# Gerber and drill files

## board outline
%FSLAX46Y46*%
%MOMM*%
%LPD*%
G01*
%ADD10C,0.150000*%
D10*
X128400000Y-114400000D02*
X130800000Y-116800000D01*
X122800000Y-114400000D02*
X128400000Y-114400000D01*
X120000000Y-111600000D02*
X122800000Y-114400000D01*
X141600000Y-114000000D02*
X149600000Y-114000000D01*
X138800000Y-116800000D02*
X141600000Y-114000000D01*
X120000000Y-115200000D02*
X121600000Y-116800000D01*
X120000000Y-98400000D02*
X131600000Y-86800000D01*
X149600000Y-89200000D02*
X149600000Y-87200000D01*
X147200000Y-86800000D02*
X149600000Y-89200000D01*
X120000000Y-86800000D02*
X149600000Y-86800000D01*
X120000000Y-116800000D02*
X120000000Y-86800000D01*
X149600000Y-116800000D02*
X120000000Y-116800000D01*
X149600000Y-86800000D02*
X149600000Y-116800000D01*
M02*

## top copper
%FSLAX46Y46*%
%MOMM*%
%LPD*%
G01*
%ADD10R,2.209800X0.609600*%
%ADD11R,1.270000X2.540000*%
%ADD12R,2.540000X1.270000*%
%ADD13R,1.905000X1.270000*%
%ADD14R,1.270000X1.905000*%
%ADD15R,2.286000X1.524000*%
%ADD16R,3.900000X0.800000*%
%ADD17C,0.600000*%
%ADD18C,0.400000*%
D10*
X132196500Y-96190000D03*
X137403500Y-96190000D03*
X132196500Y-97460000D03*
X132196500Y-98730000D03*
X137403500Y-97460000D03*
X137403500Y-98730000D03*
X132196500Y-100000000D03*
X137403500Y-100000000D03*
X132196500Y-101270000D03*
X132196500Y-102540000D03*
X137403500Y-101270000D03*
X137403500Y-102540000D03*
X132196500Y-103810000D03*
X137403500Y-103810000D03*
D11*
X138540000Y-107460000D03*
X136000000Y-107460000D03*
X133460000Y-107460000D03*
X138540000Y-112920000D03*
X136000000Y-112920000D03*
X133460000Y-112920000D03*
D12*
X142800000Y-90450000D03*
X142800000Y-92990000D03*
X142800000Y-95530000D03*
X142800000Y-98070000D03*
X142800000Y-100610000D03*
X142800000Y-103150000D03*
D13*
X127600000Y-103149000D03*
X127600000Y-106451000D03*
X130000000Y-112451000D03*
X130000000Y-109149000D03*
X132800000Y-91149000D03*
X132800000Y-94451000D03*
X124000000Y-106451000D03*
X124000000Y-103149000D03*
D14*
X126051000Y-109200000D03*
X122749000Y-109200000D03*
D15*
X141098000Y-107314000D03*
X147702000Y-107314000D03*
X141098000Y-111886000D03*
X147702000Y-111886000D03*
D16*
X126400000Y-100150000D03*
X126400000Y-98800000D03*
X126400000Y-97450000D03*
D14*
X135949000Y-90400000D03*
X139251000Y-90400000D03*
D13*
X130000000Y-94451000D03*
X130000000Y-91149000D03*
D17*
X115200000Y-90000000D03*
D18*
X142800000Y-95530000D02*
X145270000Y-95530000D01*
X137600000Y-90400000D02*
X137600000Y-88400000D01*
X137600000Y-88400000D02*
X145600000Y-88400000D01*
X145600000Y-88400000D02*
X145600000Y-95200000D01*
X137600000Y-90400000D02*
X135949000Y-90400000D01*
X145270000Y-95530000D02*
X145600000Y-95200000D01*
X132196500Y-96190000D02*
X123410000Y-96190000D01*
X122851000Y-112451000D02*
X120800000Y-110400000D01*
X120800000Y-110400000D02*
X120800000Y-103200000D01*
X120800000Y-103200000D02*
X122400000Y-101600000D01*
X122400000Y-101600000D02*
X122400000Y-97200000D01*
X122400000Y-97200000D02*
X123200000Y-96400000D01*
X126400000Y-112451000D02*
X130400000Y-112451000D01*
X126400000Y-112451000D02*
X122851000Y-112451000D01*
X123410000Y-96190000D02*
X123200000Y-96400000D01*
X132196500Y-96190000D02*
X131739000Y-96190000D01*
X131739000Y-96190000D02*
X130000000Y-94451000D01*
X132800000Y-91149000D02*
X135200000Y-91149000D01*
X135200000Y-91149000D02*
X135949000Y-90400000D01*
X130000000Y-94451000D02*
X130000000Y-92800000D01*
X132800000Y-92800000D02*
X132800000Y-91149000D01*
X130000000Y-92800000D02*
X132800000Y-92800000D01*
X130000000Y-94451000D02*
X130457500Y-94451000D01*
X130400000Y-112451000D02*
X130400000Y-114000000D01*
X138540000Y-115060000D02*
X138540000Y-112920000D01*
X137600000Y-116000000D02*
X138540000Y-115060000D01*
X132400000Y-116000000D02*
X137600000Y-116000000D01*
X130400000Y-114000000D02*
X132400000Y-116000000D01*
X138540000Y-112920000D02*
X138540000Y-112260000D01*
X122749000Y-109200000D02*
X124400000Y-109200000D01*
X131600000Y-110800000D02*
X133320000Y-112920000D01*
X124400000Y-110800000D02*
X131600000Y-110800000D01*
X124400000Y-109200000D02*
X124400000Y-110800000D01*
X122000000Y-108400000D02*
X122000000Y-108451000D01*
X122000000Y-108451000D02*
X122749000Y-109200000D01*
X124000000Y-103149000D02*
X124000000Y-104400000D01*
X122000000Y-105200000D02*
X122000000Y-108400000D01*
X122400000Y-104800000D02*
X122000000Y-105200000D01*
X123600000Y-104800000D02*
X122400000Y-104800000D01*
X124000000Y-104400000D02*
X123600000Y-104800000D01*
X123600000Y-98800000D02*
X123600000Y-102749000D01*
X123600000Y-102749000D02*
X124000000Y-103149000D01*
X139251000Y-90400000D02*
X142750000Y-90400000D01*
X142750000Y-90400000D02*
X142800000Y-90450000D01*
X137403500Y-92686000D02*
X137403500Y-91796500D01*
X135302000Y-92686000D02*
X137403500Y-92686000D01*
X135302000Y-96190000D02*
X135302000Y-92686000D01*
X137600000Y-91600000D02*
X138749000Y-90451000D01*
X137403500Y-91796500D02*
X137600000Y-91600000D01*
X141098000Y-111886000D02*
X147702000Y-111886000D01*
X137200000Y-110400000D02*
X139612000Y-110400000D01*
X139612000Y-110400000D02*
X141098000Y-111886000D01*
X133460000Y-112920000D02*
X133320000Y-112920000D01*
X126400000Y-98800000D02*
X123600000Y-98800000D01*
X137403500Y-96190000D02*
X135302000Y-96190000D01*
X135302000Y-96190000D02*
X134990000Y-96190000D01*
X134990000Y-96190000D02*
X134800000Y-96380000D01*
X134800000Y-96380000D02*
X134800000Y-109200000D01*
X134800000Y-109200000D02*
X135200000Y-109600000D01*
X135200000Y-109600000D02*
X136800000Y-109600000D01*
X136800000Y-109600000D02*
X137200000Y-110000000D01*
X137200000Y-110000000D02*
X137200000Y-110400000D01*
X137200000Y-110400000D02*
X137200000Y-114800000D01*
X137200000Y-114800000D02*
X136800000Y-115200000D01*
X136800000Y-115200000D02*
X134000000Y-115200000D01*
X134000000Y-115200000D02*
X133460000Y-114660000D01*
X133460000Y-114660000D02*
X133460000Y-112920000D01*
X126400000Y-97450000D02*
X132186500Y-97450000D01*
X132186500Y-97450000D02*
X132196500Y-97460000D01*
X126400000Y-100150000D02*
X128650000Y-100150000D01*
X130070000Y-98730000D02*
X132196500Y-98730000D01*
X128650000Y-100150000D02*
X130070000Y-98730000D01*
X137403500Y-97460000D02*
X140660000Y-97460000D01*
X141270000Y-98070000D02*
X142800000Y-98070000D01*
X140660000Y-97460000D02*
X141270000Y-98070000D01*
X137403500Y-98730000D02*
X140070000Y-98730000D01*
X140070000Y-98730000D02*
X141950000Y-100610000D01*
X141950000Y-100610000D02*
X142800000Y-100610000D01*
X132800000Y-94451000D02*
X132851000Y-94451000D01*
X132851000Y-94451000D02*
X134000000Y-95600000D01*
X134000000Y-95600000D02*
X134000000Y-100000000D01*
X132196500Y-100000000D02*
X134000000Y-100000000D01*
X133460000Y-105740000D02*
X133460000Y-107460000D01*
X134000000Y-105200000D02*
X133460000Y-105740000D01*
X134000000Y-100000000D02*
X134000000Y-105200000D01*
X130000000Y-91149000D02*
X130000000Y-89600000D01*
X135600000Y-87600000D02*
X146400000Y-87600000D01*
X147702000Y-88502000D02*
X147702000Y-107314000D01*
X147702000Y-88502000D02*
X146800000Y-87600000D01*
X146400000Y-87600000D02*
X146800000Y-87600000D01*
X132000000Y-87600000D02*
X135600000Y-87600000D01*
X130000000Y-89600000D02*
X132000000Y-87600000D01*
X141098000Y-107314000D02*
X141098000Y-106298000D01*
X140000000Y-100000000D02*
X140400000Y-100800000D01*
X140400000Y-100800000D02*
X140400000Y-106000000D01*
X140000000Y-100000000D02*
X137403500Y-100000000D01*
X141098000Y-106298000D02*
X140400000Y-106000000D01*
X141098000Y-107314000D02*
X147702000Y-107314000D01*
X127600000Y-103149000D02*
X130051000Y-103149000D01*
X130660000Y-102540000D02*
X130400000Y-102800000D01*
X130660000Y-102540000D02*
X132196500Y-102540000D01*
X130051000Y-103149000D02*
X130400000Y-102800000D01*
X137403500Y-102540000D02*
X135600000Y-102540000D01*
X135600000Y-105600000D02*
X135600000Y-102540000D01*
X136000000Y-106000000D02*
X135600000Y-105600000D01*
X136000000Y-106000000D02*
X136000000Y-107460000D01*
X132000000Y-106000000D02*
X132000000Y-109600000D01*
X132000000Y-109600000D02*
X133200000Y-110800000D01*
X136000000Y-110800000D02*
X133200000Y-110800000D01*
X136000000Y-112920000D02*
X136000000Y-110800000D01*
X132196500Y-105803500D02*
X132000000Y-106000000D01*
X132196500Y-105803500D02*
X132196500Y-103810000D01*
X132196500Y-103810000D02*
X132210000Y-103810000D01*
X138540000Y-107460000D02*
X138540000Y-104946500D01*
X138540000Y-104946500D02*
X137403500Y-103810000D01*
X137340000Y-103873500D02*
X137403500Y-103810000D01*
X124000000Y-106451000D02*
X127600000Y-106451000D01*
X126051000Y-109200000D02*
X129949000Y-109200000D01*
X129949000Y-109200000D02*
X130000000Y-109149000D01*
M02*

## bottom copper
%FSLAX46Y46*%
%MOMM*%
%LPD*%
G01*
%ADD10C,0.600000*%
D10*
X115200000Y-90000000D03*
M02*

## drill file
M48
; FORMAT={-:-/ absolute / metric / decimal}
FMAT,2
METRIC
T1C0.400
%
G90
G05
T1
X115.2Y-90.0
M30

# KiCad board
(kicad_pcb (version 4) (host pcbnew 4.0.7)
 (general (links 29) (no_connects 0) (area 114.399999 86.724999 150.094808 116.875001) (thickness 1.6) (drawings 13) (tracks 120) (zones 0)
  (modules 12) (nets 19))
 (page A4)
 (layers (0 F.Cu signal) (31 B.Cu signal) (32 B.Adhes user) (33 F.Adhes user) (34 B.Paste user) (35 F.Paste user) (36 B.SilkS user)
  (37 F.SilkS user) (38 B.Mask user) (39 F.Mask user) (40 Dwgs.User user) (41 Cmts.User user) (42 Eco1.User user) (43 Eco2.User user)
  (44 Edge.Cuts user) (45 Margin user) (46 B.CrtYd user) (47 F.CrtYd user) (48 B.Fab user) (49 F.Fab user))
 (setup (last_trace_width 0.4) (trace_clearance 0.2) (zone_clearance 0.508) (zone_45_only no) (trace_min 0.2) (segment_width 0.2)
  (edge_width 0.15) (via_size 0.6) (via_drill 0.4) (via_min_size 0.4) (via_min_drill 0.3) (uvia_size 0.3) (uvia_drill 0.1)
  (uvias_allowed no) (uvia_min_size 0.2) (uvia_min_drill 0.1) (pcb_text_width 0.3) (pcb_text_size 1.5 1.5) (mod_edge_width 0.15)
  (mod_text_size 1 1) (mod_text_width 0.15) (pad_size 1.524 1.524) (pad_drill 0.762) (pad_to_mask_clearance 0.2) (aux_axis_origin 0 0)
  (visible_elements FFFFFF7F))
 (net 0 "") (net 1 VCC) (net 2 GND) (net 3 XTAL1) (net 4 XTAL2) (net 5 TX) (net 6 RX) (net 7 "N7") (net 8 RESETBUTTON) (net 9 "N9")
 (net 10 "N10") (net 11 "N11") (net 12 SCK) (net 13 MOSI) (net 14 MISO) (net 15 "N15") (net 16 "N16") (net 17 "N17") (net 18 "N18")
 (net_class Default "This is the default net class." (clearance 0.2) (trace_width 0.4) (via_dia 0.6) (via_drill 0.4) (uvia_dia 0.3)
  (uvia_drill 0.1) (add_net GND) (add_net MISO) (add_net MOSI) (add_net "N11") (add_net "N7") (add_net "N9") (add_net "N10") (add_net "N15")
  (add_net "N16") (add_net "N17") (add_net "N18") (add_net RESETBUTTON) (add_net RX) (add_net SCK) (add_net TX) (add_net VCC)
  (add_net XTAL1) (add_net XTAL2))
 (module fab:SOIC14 (layer F.Cu) (at 134.8 100 270)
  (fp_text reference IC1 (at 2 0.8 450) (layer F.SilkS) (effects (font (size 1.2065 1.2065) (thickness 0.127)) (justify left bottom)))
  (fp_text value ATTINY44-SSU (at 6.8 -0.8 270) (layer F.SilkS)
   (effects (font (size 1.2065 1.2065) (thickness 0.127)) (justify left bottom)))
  (pad 1 smd rect (at -3.81 2.6035 270) (size 0.6096 2.2098) (layers F.Cu F.Paste F.Mask) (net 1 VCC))
  (pad 14 smd rect (at -3.81 -2.6035 270) (size 0.6096 2.2098) (layers F.Cu F.Paste F.Mask) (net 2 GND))
  (pad 2 smd rect (at -2.54 2.6035 270) (size 0.6096 2.2098) (layers F.Cu F.Paste F.Mask) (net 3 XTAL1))
  (pad 3 smd rect (at -1.27 2.6035 270) (size 0.6096 2.2098) (layers F.Cu F.Paste F.Mask) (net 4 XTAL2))
  (pad 13 smd rect (at -2.54 -2.6035 270) (size 0.6096 2.2098) (layers F.Cu F.Paste F.Mask) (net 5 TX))
  (pad 12 smd rect (at -1.27 -2.6035 270) (size 0.6096 2.2098) (layers F.Cu F.Paste F.Mask) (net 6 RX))
  (pad 4 smd rect (at 0 2.6035 270) (size 0.6096 2.2098) (layers F.Cu F.Paste F.Mask) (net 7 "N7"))
  (pad 11 smd rect (at 0 -2.6035 270) (size 0.6096 2.2098) (layers F.Cu F.Paste F.Mask) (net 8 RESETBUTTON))
  (pad 5 smd rect (at 1.27 2.6035 270) (size 0.6096 2.2098) (layers F.Cu F.Paste F.Mask) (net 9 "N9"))
  (pad 6 smd rect (at 2.54 2.6035 270) (size 0.6096 2.2098) (layers F.Cu F.Paste F.Mask) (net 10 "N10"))
  (pad 10 smd rect (at 1.27 -2.6035 270) (size 0.6096 2.2098) (layers F.Cu F.Paste F.Mask) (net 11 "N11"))
  (pad 9 smd rect (at 2.54 -2.6035 270) (size 0.6096 2.2098) (layers F.Cu F.Paste F.Mask) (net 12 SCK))
  (pad 7 smd rect (at 3.81 2.6035 270) (size 0.6096 2.2098) (layers F.Cu F.Paste F.Mask) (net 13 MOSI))
  (pad 8 smd rect (at 3.81 -2.6035 270) (size 0.6096 2.2098) (layers F.Cu F.Paste F.Mask) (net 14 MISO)))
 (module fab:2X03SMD (layer F.Cu) (at 136 110 270)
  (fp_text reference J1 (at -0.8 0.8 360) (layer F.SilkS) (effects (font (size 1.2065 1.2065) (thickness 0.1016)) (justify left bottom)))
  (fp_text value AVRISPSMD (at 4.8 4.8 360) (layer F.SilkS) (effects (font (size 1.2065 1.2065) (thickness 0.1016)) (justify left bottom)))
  (pad 1 smd rect (at -2.54 -2.54 270) (size 2.54 1.27) (layers F.Cu F.Paste F.Mask) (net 14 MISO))
  (pad 3 smd rect (at -2.54 0 270) (size 2.54 1.27) (layers F.Cu F.Paste F.Mask) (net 12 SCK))
  (pad 5 smd rect (at -2.54 2.54 270) (size 2.54 1.27) (layers F.Cu F.Paste F.Mask) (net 7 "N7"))
  (pad 2 smd rect (at 2.92 -2.54 270) (size 2.54 1.27) (layers F.Cu F.Paste F.Mask) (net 1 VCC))
  (pad 4 smd rect (at 2.92 0 270) (size 2.54 1.27) (layers F.Cu F.Paste F.Mask) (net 13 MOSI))
  (pad 6 smd rect (at 2.92 2.54 270) (size 2.54 1.27) (layers F.Cu F.Paste F.Mask) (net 2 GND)))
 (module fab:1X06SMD (layer F.Cu) (at 142.8 96.8)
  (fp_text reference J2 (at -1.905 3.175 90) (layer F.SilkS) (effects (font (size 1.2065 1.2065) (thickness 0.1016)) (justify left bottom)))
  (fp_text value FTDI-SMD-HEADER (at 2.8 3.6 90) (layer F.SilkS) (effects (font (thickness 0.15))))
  (pad 1 smd rect (at 0 -6.35) (size 2.54 1.27) (layers F.Cu F.Paste F.Mask) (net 2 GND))
  (pad 2 smd rect (at 0 -3.81) (size 2.54 1.27) (layers F.Cu F.Paste F.Mask) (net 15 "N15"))
  (pad 3 smd rect (at 0 -1.27) (size 2.54 1.27) (layers F.Cu F.Paste F.Mask) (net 1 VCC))
  (pad 4 smd rect (at 0 1.27) (size 2.54 1.27) (layers F.Cu F.Paste F.Mask) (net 5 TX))
  (pad 5 smd rect (at 0 3.81) (size 2.54 1.27) (layers F.Cu F.Paste F.Mask) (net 6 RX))
  (pad 6 smd rect (at 0 6.35) (size 2.54 1.27) (layers F.Cu F.Paste F.Mask) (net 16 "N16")))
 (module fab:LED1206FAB (layer F.Cu) (at 127.6 104.8 270)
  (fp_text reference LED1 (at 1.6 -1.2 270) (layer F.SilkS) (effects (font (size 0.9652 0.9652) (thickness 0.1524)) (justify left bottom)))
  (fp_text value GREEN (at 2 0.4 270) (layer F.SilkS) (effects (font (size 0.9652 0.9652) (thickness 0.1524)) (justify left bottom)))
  (pad 1 smd rect (at -1.651 0 270) (size 1.27 1.905) (layers F.Cu F.Paste F.Mask) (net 10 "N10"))
  (pad 2 smd rect (at 1.651 0 270) (size 1.27 1.905) (layers F.Cu F.Paste F.Mask) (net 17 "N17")))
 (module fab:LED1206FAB (layer F.Cu) (at 130 110.8 90)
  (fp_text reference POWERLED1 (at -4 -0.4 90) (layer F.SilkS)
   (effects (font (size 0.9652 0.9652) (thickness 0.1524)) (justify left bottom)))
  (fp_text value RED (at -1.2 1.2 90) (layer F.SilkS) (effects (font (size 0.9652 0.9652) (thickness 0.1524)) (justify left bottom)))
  (pad 1 smd rect (at -1.651 0 90) (size 1.27 1.905) (layers F.Cu F.Paste F.Mask) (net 1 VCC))
  (pad 2 smd rect (at 1.651 0 90) (size 1.27 1.905) (layers F.Cu F.Paste F.Mask) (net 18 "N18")))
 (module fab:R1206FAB (layer F.Cu) (at 132.8 92.8 270)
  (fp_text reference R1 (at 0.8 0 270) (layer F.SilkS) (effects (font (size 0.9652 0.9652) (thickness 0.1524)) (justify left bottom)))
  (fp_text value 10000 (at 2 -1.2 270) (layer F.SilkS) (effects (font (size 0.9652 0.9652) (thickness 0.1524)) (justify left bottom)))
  (pad 1 smd rect (at -1.651 0 270) (size 1.27 1.905) (layers F.Cu F.Paste F.Mask) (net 1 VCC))
  (pad 2 smd rect (at 1.651 0 270) (size 1.27 1.905) (layers F.Cu F.Paste F.Mask) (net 7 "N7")))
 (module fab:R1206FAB (layer F.Cu) (at 124 104.8 90)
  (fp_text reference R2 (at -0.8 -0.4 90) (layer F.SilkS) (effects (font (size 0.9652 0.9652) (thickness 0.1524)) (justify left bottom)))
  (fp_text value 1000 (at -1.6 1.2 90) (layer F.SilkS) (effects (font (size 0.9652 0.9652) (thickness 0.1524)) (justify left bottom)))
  (pad 1 smd rect (at -1.651 0 90) (size 1.27 1.905) (layers F.Cu F.Paste F.Mask) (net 17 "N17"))
  (pad 2 smd rect (at 1.651 0 90) (size 1.27 1.905) (layers F.Cu F.Paste F.Mask) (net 2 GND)))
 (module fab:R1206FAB (layer F.Cu) (at 124.4 109.2 180)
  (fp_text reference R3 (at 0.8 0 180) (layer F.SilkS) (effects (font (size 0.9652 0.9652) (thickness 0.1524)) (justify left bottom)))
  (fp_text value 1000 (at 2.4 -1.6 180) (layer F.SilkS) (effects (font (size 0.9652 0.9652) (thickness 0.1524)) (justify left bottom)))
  (pad 1 smd rect (at -1.651 0 180) (size 1.27 1.905) (layers F.Cu F.Paste F.Mask) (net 18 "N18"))
  (pad 2 smd rect (at 1.651 0 180) (size 1.27 1.905) (layers F.Cu F.Paste F.Mask) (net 2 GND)))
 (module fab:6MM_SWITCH (layer F.Cu) (at 144.4 109.6)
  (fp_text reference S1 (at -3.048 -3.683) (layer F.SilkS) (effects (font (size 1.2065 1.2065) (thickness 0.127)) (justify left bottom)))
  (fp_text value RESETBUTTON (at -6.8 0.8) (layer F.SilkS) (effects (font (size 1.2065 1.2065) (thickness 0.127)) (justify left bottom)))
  (pad 1 smd rect (at -3.302 -2.286) (size 2.286 1.524) (layers F.Cu F.Paste F.Mask) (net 8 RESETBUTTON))
  (pad 2 smd rect (at 3.302 -2.286) (size 2.286 1.524) (layers F.Cu F.Paste F.Mask) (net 8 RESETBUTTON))
  (pad 3 smd rect (at -3.302 2.286) (size 2.286 1.524) (layers F.Cu F.Paste F.Mask) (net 2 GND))
  (pad 4 smd rect (at 3.302 2.286) (size 2.286 1.524) (layers F.Cu F.Paste F.Mask) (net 2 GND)))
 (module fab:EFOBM (layer F.Cu) (at 126.4 98.8 90)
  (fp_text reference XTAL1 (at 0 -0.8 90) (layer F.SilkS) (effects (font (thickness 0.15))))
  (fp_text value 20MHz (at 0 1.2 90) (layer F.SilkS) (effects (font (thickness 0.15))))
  (pad 1 smd rect (at -1.35 0 180) (size 3.9 0.8) (layers F.Cu F.Paste F.Mask) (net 4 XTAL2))
  (pad 2 smd rect (at 0 0) (size 3.9 0.8) (layers F.Cu F.Paste F.Mask) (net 2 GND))
  (pad 3 smd rect (at 1.35 0) (size 3.9 0.8) (layers F.Cu F.Paste F.Mask) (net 3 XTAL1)))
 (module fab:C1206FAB (layer F.Cu) (at 137.6 90.4)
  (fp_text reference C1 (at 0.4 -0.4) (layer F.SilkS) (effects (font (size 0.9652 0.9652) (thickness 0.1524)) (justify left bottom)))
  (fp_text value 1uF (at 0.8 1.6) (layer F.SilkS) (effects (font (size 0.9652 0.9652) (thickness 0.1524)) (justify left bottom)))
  (pad 1 smd rect (at -1.651 0) (size 1.27 1.905) (layers F.Cu F.Paste F.Mask) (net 1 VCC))
  (pad 2 smd rect (at 1.651 0) (size 1.27 1.905) (layers F.Cu F.Paste F.Mask) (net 2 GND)))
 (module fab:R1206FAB (layer F.Cu) (at 130 92.8 90)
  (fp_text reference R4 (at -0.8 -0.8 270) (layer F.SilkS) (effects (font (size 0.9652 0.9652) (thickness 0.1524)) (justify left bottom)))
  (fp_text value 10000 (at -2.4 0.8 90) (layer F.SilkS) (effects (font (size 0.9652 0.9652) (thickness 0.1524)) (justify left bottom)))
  (pad 1 smd rect (at -1.651 0 90) (size 1.27 1.905) (layers F.Cu F.Paste F.Mask) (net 1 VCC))
  (pad 2 smd rect (at 1.651 0 90) (size 1.27 1.905) (layers F.Cu F.Paste F.Mask) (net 8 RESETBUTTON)))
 (gr_line (start 128.4 114.4) (end 130.8 116.8) (angle 90) (layer Edge.Cuts) (width 0.15))
 (gr_line (start 122.8 114.4) (end 128.4 114.4) (angle 90) (layer Edge.Cuts) (width 0.15))
 (gr_line (start 120 111.6) (end 122.8 114.4) (angle 90) (layer Edge.Cuts) (width 0.15))
 (gr_line (start 141.6 114) (end 149.6 114) (angle 90) (layer Edge.Cuts) (width 0.15))
 (gr_line (start 138.8 116.8) (end 141.6 114) (angle 90) (layer Edge.Cuts) (width 0.15))
 (gr_line (start 120 115.2) (end 121.6 116.8) (angle 90) (layer Edge.Cuts) (width 0.15))
 (gr_line (start 120 98.4) (end 131.6 86.8) (angle 90) (layer Edge.Cuts) (width 0.15))
 (gr_line (start 149.6 89.2) (end 149.6 87.2) (angle 90) (layer Edge.Cuts) (width 0.15))
 (gr_line (start 147.2 86.8) (end 149.6 89.2) (angle 90) (layer Edge.Cuts) (width 0.15))
 (gr_line (start 120 86.8) (end 149.6 86.8) (angle 90) (layer Edge.Cuts) (width 0.15))
 (gr_line (start 120 116.8) (end 120 86.8) (angle 90) (layer Edge.Cuts) (width 0.15))
 (gr_line (start 149.6 116.8) (end 120 116.8) (angle 90) (layer Edge.Cuts) (width 0.15))
 (gr_line (start 149.6 86.8) (end 149.6 116.8) (angle 90) (layer Edge.Cuts) (width 0.15))
 (via (at 115.2 90) (size 0.6) (drill 0.4) (layers F.Cu B.Cu) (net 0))
 (segment (start 142.8 95.53) (end 145.27 95.53) (width 0.4) (layer F.Cu) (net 1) (status 400000))
 (segment (start 137.6 90.4) (end 137.6 88.4) (width 0.4) (layer F.Cu) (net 1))
 (segment (start 137.6 88.4) (end 145.6 88.4) (width 0.4) (layer F.Cu) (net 1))
 (segment (start 145.6 88.4) (end 145.6 95.2) (width 0.4) (layer F.Cu) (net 1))
 (segment (start 137.6 90.4) (end 135.949 90.4) (width 0.4) (layer F.Cu) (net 1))
 (segment (start 145.27 95.53) (end 145.6 95.2) (width 0.4) (layer F.Cu) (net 1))
 (segment (start 132.1965 96.19) (end 123.41 96.19) (width 0.4) (layer F.Cu) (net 1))
 (segment (start 122.851 112.451) (end 120.8 110.4) (width 0.4) (layer F.Cu) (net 1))
 (segment (start 120.8 110.4) (end 120.8 103.2) (width 0.4) (layer F.Cu) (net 1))
 (segment (start 120.8 103.2) (end 122.4 101.6) (width 0.4) (layer F.Cu) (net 1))
 (segment (start 122.4 101.6) (end 122.4 97.2) (width 0.4) (layer F.Cu) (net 1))
 (segment (start 122.4 97.2) (end 123.2 96.4) (width 0.4) (layer F.Cu) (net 1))
 (segment (start 126.4 112.451) (end 130.4 112.451) (width 0.4) (layer F.Cu) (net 1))
 (segment (start 126.4 112.451) (end 122.851 112.451) (width 0.4) (layer F.Cu) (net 1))
 (segment (start 123.41 96.19) (end 123.2 96.4) (width 0.4) (layer F.Cu) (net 1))
 (segment (start 132.1965 96.19) (end 131.739 96.19) (width 0.4) (layer F.Cu) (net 1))
 (segment (start 131.739 96.19) (end 130 94.451) (width 0.4) (layer F.Cu) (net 1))
 (segment (start 132.8 91.149) (end 135.2 91.149) (width 0.4) (layer F.Cu) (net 1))
 (segment (start 135.2 91.149) (end 135.949 90.4) (width 0.4) (layer F.Cu) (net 1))
 (segment (start 130 94.451) (end 130 92.8) (width 0.4) (layer F.Cu) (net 1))
 (segment (start 132.8 92.8) (end 132.8 91.149) (width 0.4) (layer F.Cu) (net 1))
 (segment (start 130 92.8) (end 132.8 92.8) (width 0.4) (layer F.Cu) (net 1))
 (segment (start 130 94.451) (end 130.4575 94.451) (width 0.4) (layer F.Cu) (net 1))
 (segment (start 130.4 112.451) (end 130.4 114) (width 0.4) (layer F.Cu) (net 1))
 (segment (start 138.54 115.06) (end 138.54 112.92) (width 0.4) (layer F.Cu) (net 1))
 (segment (start 137.6 116) (end 138.54 115.06) (width 0.4) (layer F.Cu) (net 1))
 (segment (start 132.4 116) (end 137.6 116) (width 0.4) (layer F.Cu) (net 1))
 (segment (start 130.4 114) (end 132.4 116) (width 0.4) (layer F.Cu) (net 1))
 (segment (start 138.54 112.92) (end 138.54 112.26) (width 0.4) (layer F.Cu) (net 1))
 (segment (start 122.749 109.2) (end 124.4 109.2) (width 0.4) (layer F.Cu) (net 2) (status 400000))
 (segment (start 131.6 110.8) (end 133.32 112.92) (width 0.4) (layer F.Cu) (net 2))
 (segment (start 124.4 110.8) (end 131.6 110.8) (width 0.4) (layer F.Cu) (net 2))
 (segment (start 124.4 109.2) (end 124.4 110.8) (width 0.4) (layer F.Cu) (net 2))
 (segment (start 122 108.4) (end 122 108.451) (width 0.4) (layer F.Cu) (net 2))
 (segment (start 122 108.451) (end 122.749 109.2) (width 0.4) (layer F.Cu) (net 2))
 (segment (start 124 103.149) (end 124 104.4) (width 0.4) (layer F.Cu) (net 2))
 (segment (start 122 105.2) (end 122 108.4) (width 0.4) (layer F.Cu) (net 2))
 (segment (start 122.4 104.8) (end 122 105.2) (width 0.4) (layer F.Cu) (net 2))
 (segment (start 123.6 104.8) (end 122.4 104.8) (width 0.4) (layer F.Cu) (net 2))
 (segment (start 124 104.4) (end 123.6 104.8) (width 0.4) (layer F.Cu) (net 2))
 (segment (start 123.6 98.8) (end 123.6 102.749) (width 0.4) (layer F.Cu) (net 2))
 (segment (start 123.6 102.749) (end 124 103.149) (width 0.4) (layer F.Cu) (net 2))
 (segment (start 139.251 90.4) (end 142.75 90.4) (width 0.4) (layer F.Cu) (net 2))
 (segment (start 142.75 90.4) (end 142.8 90.45) (width 0.4) (layer F.Cu) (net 2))
 (segment (start 137.4035 92.686) (end 137.4035 91.7965) (width 0.4) (layer F.Cu) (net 2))
 (segment (start 135.302 92.686) (end 137.4035 92.686) (width 0.4) (layer F.Cu) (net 2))
 (segment (start 135.302 96.19) (end 135.302 92.686) (width 0.4) (layer F.Cu) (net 2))
 (segment (start 137.6 91.6) (end 138.749 90.451) (width 0.4) (layer F.Cu) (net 2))
 (segment (start 137.4035 91.7965) (end 137.6 91.6) (width 0.4) (layer F.Cu) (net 2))
 (segment (start 141.098 111.886) (end 147.702 111.886) (width 0.4) (layer F.Cu) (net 2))
 (segment (start 137.2 110.4) (end 139.612 110.4) (width 0.4) (layer F.Cu) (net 2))
 (segment (start 139.612 110.4) (end 141.098 111.886) (width 0.4) (layer F.Cu) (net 2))
 (segment (start 133.46 112.92) (end 133.32 112.92) (width 0.4) (layer F.Cu) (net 2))
 (segment (start 126.4 98.8) (end 123.6 98.8) (width 0.4) (layer F.Cu) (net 2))
 (segment (start 137.4035 96.19) (end 135.302 96.19) (width 0.4) (layer F.Cu) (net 2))
 (segment (start 135.302 96.19) (end 134.99 96.19) (width 0.4) (layer F.Cu) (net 2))
 (segment (start 134.99 96.19) (end 134.8 96.38) (width 0.4) (layer F.Cu) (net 2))
 (segment (start 134.8 96.38) (end 134.8 109.2) (width 0.4) (layer F.Cu) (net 2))
 (segment (start 134.8 109.2) (end 135.2 109.6) (width 0.4) (layer F.Cu) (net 2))
 (segment (start 135.2 109.6) (end 136.8 109.6) (width 0.4) (layer F.Cu) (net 2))
 (segment (start 136.8 109.6) (end 137.2 110) (width 0.4) (layer F.Cu) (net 2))
 (segment (start 137.2 110) (end 137.2 110.4) (width 0.4) (layer F.Cu) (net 2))
 (segment (start 137.2 110.4) (end 137.2 114.8) (width 0.4) (layer F.Cu) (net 2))
 (segment (start 137.2 114.8) (end 136.8 115.2) (width 0.4) (layer F.Cu) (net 2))
 (segment (start 136.8 115.2) (end 134 115.2) (width 0.4) (layer F.Cu) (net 2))
 (segment (start 134 115.2) (end 133.46 114.66) (width 0.4) (layer F.Cu) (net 2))
 (segment (start 133.46 114.66) (end 133.46 112.92) (width 0.4) (layer F.Cu) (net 2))
 (segment (start 126.4 97.45) (end 132.1865 97.45) (width 0.4) (layer F.Cu) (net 3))
 (segment (start 132.1865 97.45) (end 132.1965 97.46) (width 0.4) (layer F.Cu) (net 3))
 (segment (start 126.4 100.15) (end 128.65 100.15) (width 0.4) (layer F.Cu) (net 4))
 (segment (start 130.07 98.73) (end 132.1965 98.73) (width 0.4) (layer F.Cu) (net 4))
 (segment (start 128.65 100.15) (end 130.07 98.73) (width 0.4) (layer F.Cu) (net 4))
 (segment (start 137.4035 97.46) (end 140.66 97.46) (width 0.4) (layer F.Cu) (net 5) (status 400000))
 (segment (start 141.27 98.07) (end 142.8 98.07) (width 0.4) (layer F.Cu) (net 5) (status 800000))
 (segment (start 140.66 97.46) (end 141.27 98.07) (width 0.4) (layer F.Cu) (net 5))
 (segment (start 137.4035 98.73) (end 140.07 98.73) (width 0.4) (layer F.Cu) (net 6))
 (segment (start 140.07 98.73) (end 141.95 100.61) (width 0.4) (layer F.Cu) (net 6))
 (segment (start 141.95 100.61) (end 142.8 100.61) (width 0.4) (layer F.Cu) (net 6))
 (segment (start 132.8 94.451) (end 132.851 94.451) (width 0.4) (layer F.Cu) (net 7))
 (segment (start 132.851 94.451) (end 134 95.6) (width 0.4) (layer F.Cu) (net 7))
 (segment (start 134 95.6) (end 134 100) (width 0.4) (layer F.Cu) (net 7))
 (segment (start 132.1965 100) (end 134 100) (width 0.4) (layer F.Cu) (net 7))
 (segment (start 133.46 105.74) (end 133.46 107.46) (width 0.4) (layer F.Cu) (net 7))
 (segment (start 134 105.2) (end 133.46 105.74) (width 0.4) (layer F.Cu) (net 7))
 (segment (start 134 100) (end 134 105.2) (width 0.4) (layer F.Cu) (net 7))
 (segment (start 130 91.149) (end 130 89.6) (width 0.4) (layer F.Cu) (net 8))
 (segment (start 135.6 87.6) (end 146.4 87.6) (width 0.4) (layer F.Cu) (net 8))
 (segment (start 147.702 88.502) (end 147.702 107.314) (width 0.4) (layer F.Cu) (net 8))
 (segment (start 147.702 88.502) (end 146.8 87.6) (width 0.4) (layer F.Cu) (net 8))
 (segment (start 146.4 87.6) (end 146.8 87.6) (width 0.4) (layer F.Cu) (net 8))
 (segment (start 132 87.6) (end 135.6 87.6) (width 0.4) (layer F.Cu) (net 8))
 (segment (start 130 89.6) (end 132 87.6) (width 0.4) (layer F.Cu) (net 8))
 (segment (start 141.098 107.314) (end 141.098 106.298) (width 0.4) (layer F.Cu) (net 8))
 (segment (start 140 100) (end 140.4 100.8) (width 0.4) (layer F.Cu) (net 8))
 (segment (start 140.4 100.8) (end 140.4 106) (width 0.4) (layer F.Cu) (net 8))
 (segment (start 140 100) (end 137.4035 100) (width 0.4) (layer F.Cu) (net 8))
 (segment (start 141.098 106.298) (end 140.4 106) (width 0.4) (layer F.Cu) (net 8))
 (segment (start 141.098 107.314) (end 147.702 107.314) (width 0.4) (layer F.Cu) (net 8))
 (segment (start 127.6 103.149) (end 130.051 103.149) (width 0.4) (layer F.Cu) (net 10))
 (segment (start 130.66 102.54) (end 130.4 102.8) (width 0.4) (layer F.Cu) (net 10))
 (segment (start 130.66 102.54) (end 132.1965 102.54) (width 0.4) (layer F.Cu) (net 10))
 (segment (start 130.051 103.149) (end 130.4 102.8) (width 0.4) (layer F.Cu) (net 10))
 (segment (start 137.4035 102.54) (end 135.6 102.54) (width 0.4) (layer F.Cu) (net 12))
 (segment (start 135.6 105.6) (end 135.6 102.54) (width 0.4) (layer F.Cu) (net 12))
 (segment (start 136 106) (end 135.6 105.6) (width 0.4) (layer F.Cu) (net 12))
 (segment (start 136 106) (end 136 107.46) (width 0.4) (layer F.Cu) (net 12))
 (segment (start 132 106) (end 132 109.6) (width 0.4) (layer F.Cu) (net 13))
 (segment (start 132 109.6) (end 133.2 110.8) (width 0.4) (layer F.Cu) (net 13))
 (segment (start 136 110.8) (end 133.2 110.8) (width 0.4) (layer F.Cu) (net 13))
 (segment (start 136 112.92) (end 136 110.8) (width 0.4) (layer F.Cu) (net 13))
 (segment (start 132.1965 105.8035) (end 132 106) (width 0.4) (layer F.Cu) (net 13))
 (segment (start 132.1965 105.8035) (end 132.1965 103.81) (width 0.4) (layer F.Cu) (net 13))
 (segment (start 132.1965 103.81) (end 132.21 103.81) (width 0.4) (layer F.Cu) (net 13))
 (segment (start 138.54 107.46) (end 138.54 104.9465) (width 0.4) (layer F.Cu) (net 14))
 (segment (start 138.54 104.9465) (end 137.4035 103.81) (width 0.4) (layer F.Cu) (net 14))
 (segment (start 137.34 103.8735) (end 137.4035 103.81) (width 0.4) (layer F.Cu) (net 14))
 (segment (start 124 106.451) (end 127.6 106.451) (width 0.4) (layer F.Cu) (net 17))
 (segment (start 126.051 109.2) (end 129.949 109.2) (width 0.4) (layer F.Cu) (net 18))
 (segment (start 129.949 109.2) (end 130 109.149) (width 0.4) (layer F.Cu) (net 18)))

